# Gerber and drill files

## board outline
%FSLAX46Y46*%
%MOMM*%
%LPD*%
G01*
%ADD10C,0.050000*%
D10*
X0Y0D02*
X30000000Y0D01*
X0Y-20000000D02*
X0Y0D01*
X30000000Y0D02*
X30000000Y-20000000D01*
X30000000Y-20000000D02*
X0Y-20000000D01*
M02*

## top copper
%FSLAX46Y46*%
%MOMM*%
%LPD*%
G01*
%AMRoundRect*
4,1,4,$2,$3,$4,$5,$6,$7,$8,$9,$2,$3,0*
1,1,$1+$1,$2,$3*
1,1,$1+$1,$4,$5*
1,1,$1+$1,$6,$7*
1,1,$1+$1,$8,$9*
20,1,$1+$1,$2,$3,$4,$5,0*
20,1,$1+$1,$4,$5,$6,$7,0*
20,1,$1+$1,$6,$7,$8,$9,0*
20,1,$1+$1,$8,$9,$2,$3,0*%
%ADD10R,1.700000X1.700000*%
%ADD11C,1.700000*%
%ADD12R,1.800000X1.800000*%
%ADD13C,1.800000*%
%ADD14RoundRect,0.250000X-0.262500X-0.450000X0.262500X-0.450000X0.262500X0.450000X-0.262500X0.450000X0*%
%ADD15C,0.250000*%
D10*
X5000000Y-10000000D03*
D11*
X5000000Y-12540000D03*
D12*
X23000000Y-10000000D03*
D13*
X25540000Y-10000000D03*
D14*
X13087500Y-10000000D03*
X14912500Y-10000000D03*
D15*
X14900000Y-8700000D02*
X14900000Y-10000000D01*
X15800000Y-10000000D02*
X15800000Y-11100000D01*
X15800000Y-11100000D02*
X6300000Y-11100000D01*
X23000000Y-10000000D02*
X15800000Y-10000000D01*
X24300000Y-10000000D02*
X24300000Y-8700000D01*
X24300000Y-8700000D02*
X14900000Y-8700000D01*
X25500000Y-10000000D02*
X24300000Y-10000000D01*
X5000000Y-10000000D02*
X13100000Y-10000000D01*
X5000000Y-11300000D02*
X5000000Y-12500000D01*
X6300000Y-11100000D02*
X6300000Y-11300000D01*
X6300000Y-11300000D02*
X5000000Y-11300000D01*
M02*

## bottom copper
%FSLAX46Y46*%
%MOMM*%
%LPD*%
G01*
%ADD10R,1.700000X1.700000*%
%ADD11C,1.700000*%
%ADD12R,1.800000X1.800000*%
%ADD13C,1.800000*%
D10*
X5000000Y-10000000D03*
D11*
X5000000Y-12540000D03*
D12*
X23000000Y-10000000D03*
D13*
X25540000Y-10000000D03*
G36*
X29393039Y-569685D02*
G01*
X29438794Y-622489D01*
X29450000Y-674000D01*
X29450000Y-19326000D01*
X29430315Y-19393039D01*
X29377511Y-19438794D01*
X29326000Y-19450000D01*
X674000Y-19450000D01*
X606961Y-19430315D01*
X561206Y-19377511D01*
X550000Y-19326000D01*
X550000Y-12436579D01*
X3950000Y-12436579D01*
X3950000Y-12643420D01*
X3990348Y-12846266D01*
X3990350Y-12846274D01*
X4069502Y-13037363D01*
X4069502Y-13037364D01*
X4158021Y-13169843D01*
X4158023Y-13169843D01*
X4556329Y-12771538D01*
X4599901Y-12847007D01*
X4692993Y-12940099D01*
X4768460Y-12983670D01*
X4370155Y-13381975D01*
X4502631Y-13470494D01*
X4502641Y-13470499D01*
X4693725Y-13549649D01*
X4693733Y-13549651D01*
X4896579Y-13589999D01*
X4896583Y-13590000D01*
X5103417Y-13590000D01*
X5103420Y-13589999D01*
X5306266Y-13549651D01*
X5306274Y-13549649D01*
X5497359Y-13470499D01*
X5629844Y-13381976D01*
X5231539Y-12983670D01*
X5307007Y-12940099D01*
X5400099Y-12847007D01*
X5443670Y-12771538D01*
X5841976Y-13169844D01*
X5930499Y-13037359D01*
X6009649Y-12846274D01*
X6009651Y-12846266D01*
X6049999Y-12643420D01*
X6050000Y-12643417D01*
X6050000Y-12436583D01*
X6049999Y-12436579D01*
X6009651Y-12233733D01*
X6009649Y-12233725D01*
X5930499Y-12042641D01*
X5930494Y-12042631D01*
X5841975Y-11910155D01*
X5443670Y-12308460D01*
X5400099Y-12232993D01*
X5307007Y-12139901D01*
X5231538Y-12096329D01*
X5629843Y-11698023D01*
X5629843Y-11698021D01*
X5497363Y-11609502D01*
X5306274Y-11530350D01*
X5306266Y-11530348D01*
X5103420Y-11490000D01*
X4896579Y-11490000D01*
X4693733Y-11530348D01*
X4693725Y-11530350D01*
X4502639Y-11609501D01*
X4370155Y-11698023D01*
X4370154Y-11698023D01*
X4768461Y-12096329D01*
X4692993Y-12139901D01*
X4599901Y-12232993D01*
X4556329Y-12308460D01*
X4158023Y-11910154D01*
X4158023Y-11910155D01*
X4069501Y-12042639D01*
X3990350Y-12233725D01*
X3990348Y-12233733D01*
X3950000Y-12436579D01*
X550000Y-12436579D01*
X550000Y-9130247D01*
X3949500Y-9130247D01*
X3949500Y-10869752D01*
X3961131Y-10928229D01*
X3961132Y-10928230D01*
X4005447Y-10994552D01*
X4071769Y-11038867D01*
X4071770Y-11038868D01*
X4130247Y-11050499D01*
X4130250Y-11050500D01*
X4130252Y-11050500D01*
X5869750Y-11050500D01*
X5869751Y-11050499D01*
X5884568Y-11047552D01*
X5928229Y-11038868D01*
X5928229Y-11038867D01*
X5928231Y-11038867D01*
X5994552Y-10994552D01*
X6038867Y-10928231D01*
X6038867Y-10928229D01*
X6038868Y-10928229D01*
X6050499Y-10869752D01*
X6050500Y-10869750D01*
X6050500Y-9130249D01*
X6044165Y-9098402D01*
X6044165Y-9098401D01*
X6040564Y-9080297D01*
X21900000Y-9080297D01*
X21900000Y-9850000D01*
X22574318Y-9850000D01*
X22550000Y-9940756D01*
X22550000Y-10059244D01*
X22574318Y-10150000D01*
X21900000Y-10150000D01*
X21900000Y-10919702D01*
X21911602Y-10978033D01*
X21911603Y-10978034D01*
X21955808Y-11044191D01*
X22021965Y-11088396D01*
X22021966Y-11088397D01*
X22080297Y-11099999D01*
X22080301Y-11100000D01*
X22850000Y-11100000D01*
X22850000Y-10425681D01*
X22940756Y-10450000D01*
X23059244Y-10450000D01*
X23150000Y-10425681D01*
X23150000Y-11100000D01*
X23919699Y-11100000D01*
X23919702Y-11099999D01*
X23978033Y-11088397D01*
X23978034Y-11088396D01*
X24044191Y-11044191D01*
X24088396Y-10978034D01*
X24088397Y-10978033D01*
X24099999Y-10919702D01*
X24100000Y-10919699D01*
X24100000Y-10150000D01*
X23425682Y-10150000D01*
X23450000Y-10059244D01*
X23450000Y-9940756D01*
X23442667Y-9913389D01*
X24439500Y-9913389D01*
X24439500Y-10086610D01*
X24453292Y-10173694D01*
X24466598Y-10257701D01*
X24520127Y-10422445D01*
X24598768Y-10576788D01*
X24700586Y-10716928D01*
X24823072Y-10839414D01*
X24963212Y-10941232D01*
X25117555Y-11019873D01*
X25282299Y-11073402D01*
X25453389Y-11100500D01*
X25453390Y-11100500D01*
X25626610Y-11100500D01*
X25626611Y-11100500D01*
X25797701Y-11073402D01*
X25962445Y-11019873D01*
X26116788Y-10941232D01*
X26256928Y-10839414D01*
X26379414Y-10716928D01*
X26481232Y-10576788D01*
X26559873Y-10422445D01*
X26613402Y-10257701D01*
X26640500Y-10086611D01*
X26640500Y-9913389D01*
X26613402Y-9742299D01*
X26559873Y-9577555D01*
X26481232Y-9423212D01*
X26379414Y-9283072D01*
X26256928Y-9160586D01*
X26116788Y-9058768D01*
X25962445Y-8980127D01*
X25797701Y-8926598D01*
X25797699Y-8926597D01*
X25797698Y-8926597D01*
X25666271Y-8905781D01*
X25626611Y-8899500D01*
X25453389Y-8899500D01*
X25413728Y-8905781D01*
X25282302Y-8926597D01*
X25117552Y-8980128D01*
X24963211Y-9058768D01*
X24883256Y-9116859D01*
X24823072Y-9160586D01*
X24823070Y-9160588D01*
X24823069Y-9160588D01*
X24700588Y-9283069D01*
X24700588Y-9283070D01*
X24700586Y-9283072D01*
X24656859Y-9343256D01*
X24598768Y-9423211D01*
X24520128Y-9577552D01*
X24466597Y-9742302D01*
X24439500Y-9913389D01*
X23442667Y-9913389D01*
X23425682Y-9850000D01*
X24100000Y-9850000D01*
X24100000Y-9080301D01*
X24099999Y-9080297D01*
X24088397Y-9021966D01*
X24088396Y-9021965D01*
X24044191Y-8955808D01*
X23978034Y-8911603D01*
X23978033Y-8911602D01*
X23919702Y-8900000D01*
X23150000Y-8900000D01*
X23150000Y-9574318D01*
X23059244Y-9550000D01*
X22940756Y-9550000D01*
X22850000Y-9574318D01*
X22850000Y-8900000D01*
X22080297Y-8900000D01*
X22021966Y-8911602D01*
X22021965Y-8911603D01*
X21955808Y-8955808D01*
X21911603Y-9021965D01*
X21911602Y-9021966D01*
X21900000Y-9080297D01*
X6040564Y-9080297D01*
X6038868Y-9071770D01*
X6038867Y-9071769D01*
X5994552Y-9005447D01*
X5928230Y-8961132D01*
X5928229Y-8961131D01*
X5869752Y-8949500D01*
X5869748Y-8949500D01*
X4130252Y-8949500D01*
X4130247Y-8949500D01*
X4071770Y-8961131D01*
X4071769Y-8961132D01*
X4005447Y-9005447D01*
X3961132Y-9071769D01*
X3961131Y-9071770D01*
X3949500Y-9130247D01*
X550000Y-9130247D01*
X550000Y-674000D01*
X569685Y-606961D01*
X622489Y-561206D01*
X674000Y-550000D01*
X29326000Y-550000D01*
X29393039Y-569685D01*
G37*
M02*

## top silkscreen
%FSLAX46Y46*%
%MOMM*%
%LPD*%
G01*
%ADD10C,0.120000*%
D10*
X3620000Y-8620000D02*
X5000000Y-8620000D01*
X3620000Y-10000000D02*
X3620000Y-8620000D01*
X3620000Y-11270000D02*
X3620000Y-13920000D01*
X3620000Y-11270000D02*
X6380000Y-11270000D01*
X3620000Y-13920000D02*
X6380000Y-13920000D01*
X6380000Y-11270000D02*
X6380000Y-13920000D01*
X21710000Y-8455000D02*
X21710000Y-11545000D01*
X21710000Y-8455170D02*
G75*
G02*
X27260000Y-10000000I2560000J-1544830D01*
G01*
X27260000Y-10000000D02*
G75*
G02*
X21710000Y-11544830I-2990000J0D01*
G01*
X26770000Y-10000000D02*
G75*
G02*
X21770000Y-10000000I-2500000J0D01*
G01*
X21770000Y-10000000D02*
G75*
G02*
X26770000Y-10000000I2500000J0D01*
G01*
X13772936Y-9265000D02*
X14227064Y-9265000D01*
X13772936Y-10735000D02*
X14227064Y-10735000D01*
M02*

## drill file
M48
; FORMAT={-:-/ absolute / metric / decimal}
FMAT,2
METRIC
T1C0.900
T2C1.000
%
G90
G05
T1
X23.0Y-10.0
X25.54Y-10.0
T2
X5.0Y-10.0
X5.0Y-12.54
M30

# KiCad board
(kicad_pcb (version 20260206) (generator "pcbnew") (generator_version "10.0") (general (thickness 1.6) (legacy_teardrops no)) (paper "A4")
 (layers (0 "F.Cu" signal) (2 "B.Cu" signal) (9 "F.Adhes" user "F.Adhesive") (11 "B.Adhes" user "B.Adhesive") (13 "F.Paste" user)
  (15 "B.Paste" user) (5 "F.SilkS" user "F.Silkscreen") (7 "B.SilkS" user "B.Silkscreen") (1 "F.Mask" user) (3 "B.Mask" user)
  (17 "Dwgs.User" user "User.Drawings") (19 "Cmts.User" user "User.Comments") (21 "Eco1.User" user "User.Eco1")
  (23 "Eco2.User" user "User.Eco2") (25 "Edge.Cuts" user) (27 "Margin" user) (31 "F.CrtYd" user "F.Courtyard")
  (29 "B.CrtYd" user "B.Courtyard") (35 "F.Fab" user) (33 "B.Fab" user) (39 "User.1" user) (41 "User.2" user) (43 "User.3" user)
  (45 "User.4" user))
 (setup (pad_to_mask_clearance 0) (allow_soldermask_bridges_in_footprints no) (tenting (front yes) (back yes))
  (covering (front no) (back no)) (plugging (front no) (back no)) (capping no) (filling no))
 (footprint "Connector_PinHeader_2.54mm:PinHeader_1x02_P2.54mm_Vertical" (layer "F.Cu") (at 5 10)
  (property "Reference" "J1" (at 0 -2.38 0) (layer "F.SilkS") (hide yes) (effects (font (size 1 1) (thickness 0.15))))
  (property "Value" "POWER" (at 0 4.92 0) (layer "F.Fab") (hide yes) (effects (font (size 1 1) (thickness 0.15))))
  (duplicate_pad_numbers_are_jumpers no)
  (fp_line (start -1.38 -1.38) (end 0 -1.38) (stroke (width 0.12) (type solid)) (layer "F.SilkS"))
  (fp_line (start -1.38 0) (end -1.38 -1.38) (stroke (width 0.12) (type solid)) (layer "F.SilkS"))
  (fp_line (start -1.38 1.27) (end -1.38 3.92) (stroke (width 0.12) (type solid)) (layer "F.SilkS"))
  (fp_line (start -1.38 1.27) (end 1.38 1.27) (stroke (width 0.12) (type solid)) (layer "F.SilkS"))
  (fp_line (start -1.38 3.92) (end 1.38 3.92) (stroke (width 0.12) (type solid)) (layer "F.SilkS"))
  (fp_line (start 1.38 1.27) (end 1.38 3.92) (stroke (width 0.12) (type solid)) (layer "F.SilkS"))
  (pad "1" thru_hole rect (at 0 0) (size 1.7 1.7) (drill 1) (layers "*.Cu" "*.Mask") (remove_unused_layers no) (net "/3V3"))
  (pad "2" thru_hole circle (at 0 2.54) (size 1.7 1.7) (drill 1) (layers "*.Cu" "*.Mask") (remove_unused_layers no) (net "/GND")))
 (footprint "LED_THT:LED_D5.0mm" (layer "F.Cu") (at 23 10)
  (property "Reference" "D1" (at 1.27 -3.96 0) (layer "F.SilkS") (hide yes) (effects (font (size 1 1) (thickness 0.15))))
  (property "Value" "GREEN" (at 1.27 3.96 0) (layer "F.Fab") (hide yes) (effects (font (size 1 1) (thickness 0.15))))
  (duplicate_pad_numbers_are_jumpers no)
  (fp_line (start -1.29 -1.545) (end -1.29 1.545) (stroke (width 0.12) (type solid)) (layer "F.SilkS"))
  (fp_arc (start -1.29 -1.54483) (mid 2.071779 -2.880495) (end 4.26 0) (stroke (width 0.12) (type solid)) (layer "F.SilkS"))
  (fp_arc (start 4.26 0) (mid 2.071779 2.880495) (end -1.29 1.54483) (stroke (width 0.12) (type solid)) (layer "F.SilkS"))
  (fp_circle (center 1.27 0) (end 3.77 0) (stroke (width 0.12) (type solid)) (fill no) (layer "F.SilkS"))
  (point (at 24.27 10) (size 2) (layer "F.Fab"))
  (pad "1" thru_hole rect (at 0 0) (size 1.8 1.8) (drill 0.9) (layers "*.Cu" "*.Mask") (remove_unused_layers no) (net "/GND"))
  (pad "2" thru_hole circle (at 2.54 0) (size 1.8 1.8) (drill 0.9) (layers "*.Cu" "*.Mask") (remove_unused_layers no) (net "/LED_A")))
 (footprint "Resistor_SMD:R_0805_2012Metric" (layer "F.Cu") (at 14 10)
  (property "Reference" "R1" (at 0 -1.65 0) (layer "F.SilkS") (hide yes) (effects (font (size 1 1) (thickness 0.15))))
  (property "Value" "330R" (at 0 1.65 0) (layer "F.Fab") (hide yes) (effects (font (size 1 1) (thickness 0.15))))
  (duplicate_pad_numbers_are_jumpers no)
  (fp_line (start -0.227064 -0.735) (end 0.227064 -0.735) (stroke (width 0.12) (type solid)) (layer "F.SilkS"))
  (fp_line (start -0.227064 0.735) (end 0.227064 0.735) (stroke (width 0.12) (type solid)) (layer "F.SilkS"))
  (pad "1" smd roundrect (at -0.9125 0) (size 1.025 1.4) (layers "F.Cu" "F.Mask" "F.Paste") (roundrect_rratio 0.243902) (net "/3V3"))
  (pad "2" smd roundrect (at 0.9125 0) (size 1.025 1.4) (layers "F.Cu" "F.Mask" "F.Paste") (roundrect_rratio 0.243902) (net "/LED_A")))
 (gr_line (start 0 0) (end 30 0) (stroke (width 0.05) (type default)) (layer "Edge.Cuts"))
 (gr_line (start 0 20) (end 0 0) (stroke (width 0.05) (type default)) (layer "Edge.Cuts"))
 (gr_line (start 30 0) (end 30 20) (stroke (width 0.05) (type default)) (layer "Edge.Cuts"))
 (gr_line (start 30 20) (end 0 20) (stroke (width 0.05) (type default)) (layer "Edge.Cuts"))
 (segment (start 14.9 8.7) (end 14.9 10) (width 0.25) (layer "F.Cu") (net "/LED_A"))
 (segment (start 15.8 10) (end 15.8 11.1) (width 0.25) (layer "F.Cu") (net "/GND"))
 (segment (start 15.8 11.1) (end 6.3 11.1) (width 0.25) (layer "F.Cu") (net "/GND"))
 (segment (start 23 10) (end 15.8 10) (width 0.25) (layer "F.Cu") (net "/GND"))
 (segment (start 24.3 10) (end 24.3 8.7) (width 0.25) (layer "F.Cu") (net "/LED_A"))
 (segment (start 24.3 8.7) (end 14.9 8.7) (width 0.25) (layer "F.Cu") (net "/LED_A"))
 (segment (start 25.5 10) (end 24.3 10) (width 0.25) (layer "F.Cu") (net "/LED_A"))
 (segment (start 5 10) (end 13.1 10) (width 0.25) (layer "F.Cu") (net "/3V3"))
 (segment (start 5 11.3) (end 5 12.5) (width 0.25) (layer "F.Cu") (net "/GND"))
 (segment (start 6.3 11.1) (end 6.3 11.3) (width 0.25) (layer "F.Cu") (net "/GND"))
 (segment (start 6.3 11.3) (end 5 11.3) (width 0.25) (layer "F.Cu") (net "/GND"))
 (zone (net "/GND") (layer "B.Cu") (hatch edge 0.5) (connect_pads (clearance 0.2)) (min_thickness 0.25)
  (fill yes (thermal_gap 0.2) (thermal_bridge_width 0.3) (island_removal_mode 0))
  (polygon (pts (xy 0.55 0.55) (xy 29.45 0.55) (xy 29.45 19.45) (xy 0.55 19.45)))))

